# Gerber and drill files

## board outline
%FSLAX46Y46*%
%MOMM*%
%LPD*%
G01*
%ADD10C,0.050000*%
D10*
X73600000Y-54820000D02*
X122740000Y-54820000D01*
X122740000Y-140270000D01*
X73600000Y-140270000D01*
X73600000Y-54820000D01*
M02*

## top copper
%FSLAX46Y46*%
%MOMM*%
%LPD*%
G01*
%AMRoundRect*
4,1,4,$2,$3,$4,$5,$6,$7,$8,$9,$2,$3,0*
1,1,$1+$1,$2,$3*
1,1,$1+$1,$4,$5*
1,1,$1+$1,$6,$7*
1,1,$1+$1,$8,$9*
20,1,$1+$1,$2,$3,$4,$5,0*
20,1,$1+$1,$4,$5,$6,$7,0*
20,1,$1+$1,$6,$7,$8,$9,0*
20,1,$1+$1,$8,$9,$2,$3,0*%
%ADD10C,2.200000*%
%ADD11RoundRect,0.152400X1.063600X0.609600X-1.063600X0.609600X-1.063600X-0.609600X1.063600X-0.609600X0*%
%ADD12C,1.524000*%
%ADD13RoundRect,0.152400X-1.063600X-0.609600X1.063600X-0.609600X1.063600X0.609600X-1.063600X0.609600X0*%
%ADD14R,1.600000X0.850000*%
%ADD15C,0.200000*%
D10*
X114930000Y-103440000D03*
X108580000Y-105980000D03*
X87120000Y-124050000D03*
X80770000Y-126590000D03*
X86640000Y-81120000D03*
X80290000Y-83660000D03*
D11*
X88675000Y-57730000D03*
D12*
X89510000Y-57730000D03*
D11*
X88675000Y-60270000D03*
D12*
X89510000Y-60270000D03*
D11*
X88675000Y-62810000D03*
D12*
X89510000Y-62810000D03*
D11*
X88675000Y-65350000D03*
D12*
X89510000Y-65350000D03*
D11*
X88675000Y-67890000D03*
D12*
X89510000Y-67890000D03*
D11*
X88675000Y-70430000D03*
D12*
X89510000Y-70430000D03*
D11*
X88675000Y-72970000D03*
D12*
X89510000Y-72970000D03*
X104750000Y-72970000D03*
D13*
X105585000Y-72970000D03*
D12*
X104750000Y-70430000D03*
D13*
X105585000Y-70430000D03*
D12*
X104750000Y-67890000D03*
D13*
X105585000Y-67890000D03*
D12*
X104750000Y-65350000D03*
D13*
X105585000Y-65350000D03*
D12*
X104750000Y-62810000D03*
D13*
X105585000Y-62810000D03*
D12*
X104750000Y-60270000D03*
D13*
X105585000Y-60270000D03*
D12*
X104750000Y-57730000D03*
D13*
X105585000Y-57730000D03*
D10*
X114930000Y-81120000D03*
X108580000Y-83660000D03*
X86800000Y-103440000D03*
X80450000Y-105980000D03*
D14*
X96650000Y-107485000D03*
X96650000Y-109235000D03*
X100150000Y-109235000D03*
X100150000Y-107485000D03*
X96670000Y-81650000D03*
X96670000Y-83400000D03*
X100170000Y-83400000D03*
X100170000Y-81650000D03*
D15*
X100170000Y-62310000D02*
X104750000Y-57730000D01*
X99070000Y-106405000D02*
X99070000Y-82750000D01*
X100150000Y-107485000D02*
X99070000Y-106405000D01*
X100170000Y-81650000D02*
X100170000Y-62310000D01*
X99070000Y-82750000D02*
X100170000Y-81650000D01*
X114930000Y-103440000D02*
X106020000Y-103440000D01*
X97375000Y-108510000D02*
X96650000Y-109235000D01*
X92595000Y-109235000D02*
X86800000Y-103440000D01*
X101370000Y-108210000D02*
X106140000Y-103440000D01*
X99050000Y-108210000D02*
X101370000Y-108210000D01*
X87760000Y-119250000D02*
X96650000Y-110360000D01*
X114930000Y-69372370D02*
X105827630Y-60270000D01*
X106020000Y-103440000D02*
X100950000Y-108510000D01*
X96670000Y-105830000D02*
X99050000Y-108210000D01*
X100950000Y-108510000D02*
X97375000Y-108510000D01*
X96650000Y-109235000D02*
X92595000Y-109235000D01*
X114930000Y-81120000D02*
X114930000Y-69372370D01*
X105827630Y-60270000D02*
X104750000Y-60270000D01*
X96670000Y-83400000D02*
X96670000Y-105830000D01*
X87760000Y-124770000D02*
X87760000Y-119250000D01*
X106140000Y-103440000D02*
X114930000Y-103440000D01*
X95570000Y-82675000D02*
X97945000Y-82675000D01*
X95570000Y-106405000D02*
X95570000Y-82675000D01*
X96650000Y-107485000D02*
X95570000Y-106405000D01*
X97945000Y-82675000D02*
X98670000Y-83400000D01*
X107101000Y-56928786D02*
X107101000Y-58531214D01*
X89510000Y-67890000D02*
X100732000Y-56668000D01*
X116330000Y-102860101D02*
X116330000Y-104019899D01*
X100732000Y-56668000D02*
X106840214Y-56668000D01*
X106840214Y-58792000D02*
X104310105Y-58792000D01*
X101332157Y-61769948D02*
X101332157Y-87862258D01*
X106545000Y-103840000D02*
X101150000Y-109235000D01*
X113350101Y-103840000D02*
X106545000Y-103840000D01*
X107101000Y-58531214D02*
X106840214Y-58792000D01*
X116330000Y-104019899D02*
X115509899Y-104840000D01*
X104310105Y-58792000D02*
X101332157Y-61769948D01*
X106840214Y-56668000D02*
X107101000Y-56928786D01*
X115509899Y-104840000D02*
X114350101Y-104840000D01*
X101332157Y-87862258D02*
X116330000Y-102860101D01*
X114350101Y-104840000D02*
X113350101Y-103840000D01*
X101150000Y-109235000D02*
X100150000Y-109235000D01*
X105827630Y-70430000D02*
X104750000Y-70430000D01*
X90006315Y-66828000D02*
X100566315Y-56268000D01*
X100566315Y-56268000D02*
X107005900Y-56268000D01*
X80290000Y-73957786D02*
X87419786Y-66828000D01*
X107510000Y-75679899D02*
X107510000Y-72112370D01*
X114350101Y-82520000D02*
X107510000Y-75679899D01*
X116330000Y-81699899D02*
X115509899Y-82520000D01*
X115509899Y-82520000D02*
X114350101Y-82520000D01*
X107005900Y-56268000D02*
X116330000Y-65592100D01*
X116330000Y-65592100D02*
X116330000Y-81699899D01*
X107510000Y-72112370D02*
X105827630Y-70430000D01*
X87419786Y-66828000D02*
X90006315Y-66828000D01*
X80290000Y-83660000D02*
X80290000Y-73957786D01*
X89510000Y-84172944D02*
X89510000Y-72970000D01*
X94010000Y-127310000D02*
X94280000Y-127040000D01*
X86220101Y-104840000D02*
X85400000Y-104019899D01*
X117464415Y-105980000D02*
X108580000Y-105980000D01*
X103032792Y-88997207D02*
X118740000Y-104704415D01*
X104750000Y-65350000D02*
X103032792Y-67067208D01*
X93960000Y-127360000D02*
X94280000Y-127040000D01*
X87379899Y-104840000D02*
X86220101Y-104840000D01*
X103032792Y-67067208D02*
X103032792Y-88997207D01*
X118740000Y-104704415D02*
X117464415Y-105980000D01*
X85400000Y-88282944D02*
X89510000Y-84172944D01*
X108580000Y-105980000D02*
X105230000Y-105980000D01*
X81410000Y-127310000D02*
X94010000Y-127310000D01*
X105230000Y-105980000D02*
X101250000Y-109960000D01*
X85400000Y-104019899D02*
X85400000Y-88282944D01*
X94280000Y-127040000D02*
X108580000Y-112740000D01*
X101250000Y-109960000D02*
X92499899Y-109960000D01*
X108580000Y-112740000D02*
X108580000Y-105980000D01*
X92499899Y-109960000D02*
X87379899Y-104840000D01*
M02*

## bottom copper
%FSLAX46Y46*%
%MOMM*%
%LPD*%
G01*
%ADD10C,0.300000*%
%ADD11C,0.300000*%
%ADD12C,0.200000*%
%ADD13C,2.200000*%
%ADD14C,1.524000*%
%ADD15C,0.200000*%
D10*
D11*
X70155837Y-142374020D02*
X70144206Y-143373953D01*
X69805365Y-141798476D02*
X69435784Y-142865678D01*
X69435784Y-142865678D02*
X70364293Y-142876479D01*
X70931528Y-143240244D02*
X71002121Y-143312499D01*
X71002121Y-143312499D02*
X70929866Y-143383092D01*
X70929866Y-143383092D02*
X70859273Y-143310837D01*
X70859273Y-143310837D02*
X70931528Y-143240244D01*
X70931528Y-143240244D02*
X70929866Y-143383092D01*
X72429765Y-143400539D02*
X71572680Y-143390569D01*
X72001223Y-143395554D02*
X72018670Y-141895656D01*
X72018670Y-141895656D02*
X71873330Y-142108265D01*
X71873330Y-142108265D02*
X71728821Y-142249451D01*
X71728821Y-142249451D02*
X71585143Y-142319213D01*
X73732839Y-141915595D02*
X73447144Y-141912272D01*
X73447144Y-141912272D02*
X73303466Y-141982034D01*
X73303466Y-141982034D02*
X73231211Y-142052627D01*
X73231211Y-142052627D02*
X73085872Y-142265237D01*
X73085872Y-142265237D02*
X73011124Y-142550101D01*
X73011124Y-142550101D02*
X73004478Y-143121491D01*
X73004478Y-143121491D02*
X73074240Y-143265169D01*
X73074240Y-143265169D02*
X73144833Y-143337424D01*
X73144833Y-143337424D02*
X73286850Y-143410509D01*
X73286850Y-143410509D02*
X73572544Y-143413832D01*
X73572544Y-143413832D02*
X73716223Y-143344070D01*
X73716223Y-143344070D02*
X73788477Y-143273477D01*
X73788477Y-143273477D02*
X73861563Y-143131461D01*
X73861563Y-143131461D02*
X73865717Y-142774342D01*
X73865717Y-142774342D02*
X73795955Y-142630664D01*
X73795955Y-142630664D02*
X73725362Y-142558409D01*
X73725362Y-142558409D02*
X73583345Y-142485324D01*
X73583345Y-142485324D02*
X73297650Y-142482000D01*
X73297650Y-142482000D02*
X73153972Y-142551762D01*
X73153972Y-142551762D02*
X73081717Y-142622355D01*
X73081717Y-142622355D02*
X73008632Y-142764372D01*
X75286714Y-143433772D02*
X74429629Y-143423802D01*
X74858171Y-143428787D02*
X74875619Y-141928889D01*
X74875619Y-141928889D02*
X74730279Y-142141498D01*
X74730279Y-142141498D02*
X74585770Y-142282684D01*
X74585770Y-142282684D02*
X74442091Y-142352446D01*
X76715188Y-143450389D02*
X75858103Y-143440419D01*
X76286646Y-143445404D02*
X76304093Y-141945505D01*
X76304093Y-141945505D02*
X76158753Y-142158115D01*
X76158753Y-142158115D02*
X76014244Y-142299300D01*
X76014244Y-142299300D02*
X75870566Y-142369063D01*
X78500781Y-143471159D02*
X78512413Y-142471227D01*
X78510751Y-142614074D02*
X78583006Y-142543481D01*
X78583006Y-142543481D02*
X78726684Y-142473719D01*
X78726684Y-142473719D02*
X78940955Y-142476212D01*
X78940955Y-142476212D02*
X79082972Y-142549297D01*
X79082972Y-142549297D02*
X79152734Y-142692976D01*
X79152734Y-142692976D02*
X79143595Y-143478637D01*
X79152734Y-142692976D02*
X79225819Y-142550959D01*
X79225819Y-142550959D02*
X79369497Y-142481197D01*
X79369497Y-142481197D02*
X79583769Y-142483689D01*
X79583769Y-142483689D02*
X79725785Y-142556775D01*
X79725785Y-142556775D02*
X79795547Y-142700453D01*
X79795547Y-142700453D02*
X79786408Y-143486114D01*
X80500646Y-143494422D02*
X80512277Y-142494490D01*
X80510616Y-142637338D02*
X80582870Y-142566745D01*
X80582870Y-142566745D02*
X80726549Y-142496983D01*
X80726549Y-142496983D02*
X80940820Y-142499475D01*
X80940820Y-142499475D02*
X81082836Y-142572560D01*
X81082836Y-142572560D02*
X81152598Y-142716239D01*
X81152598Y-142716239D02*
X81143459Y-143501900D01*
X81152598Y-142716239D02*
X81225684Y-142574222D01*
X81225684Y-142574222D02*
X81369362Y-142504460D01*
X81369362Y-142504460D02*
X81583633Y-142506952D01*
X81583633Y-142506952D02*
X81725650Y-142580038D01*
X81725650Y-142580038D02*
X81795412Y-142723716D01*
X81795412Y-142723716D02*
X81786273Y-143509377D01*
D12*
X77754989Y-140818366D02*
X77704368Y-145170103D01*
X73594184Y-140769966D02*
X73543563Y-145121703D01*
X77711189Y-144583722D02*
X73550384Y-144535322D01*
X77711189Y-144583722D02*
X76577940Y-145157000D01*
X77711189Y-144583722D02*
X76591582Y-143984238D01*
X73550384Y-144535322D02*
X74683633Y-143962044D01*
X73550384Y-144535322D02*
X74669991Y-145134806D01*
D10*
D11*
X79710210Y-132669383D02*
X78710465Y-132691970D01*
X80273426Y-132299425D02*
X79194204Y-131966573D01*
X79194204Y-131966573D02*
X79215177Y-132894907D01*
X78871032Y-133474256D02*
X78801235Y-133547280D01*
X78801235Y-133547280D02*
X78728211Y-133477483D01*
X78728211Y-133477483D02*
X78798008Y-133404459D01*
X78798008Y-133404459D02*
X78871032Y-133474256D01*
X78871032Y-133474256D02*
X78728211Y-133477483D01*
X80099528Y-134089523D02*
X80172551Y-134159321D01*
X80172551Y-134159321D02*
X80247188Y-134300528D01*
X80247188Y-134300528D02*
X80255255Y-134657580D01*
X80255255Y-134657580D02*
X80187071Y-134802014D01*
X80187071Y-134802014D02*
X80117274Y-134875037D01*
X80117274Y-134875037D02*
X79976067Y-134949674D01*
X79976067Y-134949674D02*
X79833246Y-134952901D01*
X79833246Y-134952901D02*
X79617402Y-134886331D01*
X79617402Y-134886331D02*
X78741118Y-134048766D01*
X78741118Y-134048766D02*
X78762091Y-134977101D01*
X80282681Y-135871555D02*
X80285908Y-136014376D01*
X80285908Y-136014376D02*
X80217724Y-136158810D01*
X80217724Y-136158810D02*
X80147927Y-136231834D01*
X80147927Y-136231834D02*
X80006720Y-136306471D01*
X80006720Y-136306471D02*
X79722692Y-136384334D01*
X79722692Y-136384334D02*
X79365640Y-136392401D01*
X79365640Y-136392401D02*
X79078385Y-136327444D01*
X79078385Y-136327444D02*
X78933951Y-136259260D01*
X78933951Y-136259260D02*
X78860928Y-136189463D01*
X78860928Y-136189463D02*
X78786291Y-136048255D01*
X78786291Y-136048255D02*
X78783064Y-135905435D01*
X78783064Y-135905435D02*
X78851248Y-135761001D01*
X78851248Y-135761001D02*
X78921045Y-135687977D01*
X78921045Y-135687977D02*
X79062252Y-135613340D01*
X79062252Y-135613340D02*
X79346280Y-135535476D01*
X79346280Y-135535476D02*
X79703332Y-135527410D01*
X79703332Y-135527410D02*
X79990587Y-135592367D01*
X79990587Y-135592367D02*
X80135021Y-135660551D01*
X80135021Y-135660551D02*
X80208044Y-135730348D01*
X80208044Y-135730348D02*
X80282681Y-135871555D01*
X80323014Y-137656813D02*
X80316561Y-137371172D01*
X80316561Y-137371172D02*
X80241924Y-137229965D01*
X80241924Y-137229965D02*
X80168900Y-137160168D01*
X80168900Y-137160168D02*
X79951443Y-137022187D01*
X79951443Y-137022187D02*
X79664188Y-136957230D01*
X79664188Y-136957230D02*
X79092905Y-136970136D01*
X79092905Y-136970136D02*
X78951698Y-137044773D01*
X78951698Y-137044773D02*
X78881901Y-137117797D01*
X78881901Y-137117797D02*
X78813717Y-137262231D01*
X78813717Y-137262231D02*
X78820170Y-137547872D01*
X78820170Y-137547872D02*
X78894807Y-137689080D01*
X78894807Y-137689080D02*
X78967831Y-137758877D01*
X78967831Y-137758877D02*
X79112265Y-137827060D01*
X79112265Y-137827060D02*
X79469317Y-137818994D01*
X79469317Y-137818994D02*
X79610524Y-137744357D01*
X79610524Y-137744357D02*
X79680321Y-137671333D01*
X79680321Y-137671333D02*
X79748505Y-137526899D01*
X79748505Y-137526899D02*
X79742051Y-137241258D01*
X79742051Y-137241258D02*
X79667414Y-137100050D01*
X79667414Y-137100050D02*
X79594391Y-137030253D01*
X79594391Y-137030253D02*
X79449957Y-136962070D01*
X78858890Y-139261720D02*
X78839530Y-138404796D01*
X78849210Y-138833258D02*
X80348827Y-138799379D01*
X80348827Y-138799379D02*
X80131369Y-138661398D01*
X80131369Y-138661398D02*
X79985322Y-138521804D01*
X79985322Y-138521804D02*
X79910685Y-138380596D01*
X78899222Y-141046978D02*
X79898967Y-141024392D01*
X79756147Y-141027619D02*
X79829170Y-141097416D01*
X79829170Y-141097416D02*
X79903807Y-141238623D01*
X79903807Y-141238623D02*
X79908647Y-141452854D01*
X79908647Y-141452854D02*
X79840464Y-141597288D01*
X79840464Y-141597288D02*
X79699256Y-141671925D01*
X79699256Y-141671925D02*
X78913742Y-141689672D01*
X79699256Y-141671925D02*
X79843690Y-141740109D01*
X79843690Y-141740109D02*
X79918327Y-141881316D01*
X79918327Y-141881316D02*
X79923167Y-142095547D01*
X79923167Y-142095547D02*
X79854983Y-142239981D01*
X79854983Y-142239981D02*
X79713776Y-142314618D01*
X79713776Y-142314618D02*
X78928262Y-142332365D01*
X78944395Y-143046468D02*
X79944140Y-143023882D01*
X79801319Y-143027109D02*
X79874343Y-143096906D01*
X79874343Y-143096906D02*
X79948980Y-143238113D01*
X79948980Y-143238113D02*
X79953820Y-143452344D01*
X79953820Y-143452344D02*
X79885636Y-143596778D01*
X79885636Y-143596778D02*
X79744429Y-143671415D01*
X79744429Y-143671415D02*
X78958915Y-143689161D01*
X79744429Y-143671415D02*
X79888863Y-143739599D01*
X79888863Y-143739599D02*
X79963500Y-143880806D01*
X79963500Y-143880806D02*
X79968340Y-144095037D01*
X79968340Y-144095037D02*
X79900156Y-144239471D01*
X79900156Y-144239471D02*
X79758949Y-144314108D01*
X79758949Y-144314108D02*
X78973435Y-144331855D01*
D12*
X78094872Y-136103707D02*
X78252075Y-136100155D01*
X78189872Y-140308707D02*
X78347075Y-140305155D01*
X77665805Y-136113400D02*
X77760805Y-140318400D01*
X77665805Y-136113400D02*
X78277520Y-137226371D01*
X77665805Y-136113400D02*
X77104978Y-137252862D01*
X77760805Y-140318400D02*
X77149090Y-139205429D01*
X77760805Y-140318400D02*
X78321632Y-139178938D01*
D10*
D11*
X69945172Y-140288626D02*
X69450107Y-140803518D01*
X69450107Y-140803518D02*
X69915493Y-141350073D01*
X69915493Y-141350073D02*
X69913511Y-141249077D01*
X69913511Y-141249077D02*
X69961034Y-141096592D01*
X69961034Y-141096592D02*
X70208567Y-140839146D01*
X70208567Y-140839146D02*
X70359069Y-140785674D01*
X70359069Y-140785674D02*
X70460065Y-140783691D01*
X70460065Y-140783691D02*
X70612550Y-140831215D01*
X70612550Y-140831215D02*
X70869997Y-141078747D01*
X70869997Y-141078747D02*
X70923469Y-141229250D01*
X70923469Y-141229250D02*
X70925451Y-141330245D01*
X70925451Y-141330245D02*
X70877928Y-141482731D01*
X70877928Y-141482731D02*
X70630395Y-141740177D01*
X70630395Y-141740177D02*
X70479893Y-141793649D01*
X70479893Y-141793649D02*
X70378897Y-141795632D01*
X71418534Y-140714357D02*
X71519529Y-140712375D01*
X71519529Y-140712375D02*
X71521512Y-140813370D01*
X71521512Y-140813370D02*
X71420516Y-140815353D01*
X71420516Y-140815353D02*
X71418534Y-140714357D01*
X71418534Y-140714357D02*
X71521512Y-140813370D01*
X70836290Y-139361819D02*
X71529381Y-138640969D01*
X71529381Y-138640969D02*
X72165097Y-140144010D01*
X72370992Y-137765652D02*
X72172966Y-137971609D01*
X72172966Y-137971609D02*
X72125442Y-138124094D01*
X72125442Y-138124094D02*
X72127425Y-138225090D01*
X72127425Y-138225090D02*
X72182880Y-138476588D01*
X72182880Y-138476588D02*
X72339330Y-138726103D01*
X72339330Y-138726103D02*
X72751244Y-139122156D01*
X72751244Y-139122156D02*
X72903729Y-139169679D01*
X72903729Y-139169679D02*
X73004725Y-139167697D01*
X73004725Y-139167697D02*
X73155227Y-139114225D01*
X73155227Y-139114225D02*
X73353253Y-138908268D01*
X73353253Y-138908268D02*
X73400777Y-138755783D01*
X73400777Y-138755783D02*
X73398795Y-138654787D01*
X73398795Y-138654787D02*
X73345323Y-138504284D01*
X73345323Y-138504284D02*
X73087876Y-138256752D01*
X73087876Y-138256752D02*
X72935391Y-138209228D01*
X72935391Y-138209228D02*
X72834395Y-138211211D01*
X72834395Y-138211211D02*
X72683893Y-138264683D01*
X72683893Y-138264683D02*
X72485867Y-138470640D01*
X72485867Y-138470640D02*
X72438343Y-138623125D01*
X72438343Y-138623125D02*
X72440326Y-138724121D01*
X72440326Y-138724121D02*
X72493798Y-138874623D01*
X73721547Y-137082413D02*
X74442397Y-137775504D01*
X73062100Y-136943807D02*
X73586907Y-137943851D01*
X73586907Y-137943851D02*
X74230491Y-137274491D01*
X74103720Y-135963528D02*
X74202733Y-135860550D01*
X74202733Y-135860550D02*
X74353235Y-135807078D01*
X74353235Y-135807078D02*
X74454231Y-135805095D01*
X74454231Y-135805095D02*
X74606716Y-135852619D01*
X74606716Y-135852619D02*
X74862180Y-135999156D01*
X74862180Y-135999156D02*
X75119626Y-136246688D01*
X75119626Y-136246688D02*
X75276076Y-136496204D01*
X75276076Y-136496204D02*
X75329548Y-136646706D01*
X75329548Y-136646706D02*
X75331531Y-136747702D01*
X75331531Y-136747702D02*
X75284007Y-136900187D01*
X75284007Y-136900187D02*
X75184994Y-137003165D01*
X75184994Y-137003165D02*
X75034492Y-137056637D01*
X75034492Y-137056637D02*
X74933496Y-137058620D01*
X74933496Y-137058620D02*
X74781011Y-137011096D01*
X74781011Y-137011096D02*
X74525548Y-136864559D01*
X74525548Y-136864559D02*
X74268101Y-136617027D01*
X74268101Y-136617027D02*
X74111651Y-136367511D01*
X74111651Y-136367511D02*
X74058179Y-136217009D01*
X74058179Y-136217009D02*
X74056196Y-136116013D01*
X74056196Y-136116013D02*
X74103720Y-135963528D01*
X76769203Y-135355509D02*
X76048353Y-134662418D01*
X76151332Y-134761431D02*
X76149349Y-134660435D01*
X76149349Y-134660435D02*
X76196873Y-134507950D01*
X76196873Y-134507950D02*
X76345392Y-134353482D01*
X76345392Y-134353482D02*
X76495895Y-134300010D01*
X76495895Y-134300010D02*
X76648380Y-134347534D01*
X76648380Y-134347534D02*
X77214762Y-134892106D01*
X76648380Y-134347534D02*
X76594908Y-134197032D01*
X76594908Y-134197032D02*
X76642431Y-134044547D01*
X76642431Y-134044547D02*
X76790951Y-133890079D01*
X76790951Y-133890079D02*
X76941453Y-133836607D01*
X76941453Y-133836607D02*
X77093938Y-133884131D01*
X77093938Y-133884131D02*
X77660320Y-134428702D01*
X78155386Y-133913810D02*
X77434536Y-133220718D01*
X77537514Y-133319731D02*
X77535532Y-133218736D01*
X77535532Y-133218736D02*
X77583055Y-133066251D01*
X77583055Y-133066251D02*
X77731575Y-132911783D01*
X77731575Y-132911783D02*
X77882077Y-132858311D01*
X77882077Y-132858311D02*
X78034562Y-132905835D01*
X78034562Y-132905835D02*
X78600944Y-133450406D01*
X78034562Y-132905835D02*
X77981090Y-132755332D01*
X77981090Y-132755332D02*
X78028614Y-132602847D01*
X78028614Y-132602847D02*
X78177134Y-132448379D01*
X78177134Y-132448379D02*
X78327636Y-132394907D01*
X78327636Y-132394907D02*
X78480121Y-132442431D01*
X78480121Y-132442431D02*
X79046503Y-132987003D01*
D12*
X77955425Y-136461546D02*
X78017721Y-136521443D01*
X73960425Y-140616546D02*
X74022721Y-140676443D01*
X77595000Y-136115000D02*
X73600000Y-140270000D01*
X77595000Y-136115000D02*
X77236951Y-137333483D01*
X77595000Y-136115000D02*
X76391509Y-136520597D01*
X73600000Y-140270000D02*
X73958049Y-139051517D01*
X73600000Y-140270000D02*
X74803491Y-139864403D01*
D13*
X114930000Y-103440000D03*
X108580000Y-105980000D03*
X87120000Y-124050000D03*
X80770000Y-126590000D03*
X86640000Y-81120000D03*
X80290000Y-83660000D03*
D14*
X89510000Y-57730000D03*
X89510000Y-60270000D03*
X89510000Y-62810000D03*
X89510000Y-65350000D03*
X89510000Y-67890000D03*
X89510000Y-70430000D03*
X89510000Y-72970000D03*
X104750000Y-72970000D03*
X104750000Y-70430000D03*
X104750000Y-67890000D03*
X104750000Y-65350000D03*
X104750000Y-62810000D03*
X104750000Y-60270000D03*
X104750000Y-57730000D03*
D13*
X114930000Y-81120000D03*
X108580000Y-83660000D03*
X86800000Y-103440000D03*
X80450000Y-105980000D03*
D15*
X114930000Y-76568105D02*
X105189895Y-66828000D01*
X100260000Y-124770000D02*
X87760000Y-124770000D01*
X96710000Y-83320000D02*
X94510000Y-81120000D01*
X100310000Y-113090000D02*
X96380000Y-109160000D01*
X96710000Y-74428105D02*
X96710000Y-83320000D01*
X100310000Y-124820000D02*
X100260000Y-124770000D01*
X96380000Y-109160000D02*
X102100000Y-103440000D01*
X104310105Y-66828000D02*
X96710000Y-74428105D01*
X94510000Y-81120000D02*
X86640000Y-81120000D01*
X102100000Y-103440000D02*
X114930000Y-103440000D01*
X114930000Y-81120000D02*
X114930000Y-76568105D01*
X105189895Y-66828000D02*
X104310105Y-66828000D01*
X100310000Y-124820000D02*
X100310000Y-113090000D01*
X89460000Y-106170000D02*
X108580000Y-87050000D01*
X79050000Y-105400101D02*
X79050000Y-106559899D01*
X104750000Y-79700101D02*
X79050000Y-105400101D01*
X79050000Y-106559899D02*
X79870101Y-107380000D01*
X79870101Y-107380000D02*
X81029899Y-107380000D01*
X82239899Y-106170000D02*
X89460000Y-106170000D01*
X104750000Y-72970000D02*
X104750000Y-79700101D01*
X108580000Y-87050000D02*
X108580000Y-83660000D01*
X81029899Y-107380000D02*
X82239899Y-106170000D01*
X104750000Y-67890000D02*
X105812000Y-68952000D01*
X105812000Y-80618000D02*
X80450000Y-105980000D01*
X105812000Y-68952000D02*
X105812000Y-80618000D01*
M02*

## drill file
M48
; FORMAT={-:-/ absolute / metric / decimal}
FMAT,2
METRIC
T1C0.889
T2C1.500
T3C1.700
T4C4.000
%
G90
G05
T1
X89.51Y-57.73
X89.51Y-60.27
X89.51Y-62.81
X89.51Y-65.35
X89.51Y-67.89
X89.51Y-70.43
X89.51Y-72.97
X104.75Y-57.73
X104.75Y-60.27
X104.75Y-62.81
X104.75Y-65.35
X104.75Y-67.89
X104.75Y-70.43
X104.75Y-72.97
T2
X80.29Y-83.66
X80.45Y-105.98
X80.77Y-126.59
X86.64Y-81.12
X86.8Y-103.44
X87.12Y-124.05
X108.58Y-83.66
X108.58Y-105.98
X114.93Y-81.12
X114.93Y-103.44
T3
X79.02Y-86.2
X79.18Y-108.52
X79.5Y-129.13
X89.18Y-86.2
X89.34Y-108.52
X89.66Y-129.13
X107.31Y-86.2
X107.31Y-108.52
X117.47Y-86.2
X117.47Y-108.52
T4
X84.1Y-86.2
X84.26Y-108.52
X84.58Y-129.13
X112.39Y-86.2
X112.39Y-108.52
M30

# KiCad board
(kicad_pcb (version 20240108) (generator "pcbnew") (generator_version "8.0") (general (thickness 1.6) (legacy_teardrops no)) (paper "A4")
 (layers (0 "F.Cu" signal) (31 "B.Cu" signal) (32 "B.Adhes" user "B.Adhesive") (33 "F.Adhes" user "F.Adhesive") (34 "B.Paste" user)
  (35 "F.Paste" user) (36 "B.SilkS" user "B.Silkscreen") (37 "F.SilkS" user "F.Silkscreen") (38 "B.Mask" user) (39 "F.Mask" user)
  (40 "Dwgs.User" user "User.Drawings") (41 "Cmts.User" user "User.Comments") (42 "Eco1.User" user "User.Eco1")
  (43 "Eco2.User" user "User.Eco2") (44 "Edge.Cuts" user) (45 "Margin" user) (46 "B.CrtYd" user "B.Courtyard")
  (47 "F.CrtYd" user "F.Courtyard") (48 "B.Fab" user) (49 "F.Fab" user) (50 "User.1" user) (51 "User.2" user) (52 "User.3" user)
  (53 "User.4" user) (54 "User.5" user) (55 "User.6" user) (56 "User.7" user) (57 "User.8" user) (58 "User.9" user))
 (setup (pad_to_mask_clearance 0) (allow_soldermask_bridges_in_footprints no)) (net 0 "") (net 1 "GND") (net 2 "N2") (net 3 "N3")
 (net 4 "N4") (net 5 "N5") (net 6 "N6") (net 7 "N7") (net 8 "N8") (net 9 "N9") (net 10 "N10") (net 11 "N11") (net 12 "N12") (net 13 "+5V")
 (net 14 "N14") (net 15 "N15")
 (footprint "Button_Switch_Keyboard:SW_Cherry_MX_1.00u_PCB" (layer "F.Cu") (at 114.93 103.44)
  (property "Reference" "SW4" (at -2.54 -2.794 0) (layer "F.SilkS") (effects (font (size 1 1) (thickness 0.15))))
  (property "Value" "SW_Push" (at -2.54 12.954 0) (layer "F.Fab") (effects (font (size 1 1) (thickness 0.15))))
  (pad "" np_thru_hole circle (at -7.62 5.08) (size 1.7 1.7) (drill 1.7) (layers "*.Cu" "*.Mask"))
  (pad "" np_thru_hole circle (at -2.54 5.08) (size 4 4) (drill 4) (layers "*.Cu" "*.Mask"))
  (pad "" np_thru_hole circle (at 2.54 5.08) (size 1.7 1.7) (drill 1.7) (layers "*.Cu" "*.Mask"))
  (pad "1" thru_hole circle (at 0 0) (size 2.2 2.2) (drill 1.5) (layers "*.Cu" "*.Mask") (remove_unused_layers no) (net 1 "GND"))
  (pad "2" thru_hole circle (at -6.35 2.54) (size 2.2 2.2) (drill 1.5) (layers "*.Cu" "*.Mask") (remove_unused_layers no) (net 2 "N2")))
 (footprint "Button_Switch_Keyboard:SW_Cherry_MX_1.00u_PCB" (layer "F.Cu") (at 87.12 124.05)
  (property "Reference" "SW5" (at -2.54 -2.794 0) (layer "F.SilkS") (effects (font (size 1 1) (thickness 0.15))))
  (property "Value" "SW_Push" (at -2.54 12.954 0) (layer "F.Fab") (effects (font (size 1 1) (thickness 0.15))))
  (pad "" np_thru_hole circle (at -7.62 5.08) (size 1.7 1.7) (drill 1.7) (layers "*.Cu" "*.Mask"))
  (pad "" np_thru_hole circle (at -2.54 5.08) (size 4 4) (drill 4) (layers "*.Cu" "*.Mask"))
  (pad "" np_thru_hole circle (at 2.54 5.08) (size 1.7 1.7) (drill 1.7) (layers "*.Cu" "*.Mask"))
  (pad "1" thru_hole circle (at 0 0) (size 2.2 2.2) (drill 1.5) (layers "*.Cu" "*.Mask") (remove_unused_layers no) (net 1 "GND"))
  (pad "2" thru_hole circle (at -6.35 2.54) (size 2.2 2.2) (drill 1.5) (layers "*.Cu" "*.Mask") (remove_unused_layers no) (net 2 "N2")))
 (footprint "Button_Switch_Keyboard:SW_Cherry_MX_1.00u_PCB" (layer "F.Cu") (at 86.64 81.12)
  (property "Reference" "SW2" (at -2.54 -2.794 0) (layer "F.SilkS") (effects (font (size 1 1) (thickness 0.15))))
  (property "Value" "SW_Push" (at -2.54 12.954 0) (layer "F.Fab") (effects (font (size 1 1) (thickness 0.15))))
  (pad "" np_thru_hole circle (at -7.62 5.08) (size 1.7 1.7) (drill 1.7) (layers "*.Cu" "*.Mask"))
  (pad "" np_thru_hole circle (at -2.54 5.08) (size 4 4) (drill 4) (layers "*.Cu" "*.Mask"))
  (pad "" np_thru_hole circle (at 2.54 5.08) (size 1.7 1.7) (drill 1.7) (layers "*.Cu" "*.Mask"))
  (pad "1" thru_hole circle (at 0 0) (size 2.2 2.2) (drill 1.5) (layers "*.Cu" "*.Mask") (remove_unused_layers no) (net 1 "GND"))
  (pad "2" thru_hole circle (at -6.35 2.54) (size 2.2 2.2) (drill 1.5) (layers "*.Cu" "*.Mask") (remove_unused_layers no) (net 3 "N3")))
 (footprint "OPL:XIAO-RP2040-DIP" (layer "F.Cu") (at 97.13 65.35)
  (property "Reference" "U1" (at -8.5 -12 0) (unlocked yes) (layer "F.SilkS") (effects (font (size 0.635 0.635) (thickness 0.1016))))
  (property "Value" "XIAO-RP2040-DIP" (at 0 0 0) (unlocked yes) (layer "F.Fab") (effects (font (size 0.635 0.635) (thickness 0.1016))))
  (pad "1" smd roundrect (at -8.455 -7.62 180) (size 2.432 1.524) (layers "F.Cu" "F.Mask") (roundrect_rratio 0.1) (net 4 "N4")
   (thermal_bridge_angle 45))
  (pad "1" thru_hole circle (at -7.62 -7.62 180) (size 1.524 1.524) (drill 0.889) (layers "*.Cu" "*.Mask") (remove_unused_layers no)
   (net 4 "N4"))
  (pad "2" smd roundrect (at -8.455 -5.08 180) (size 2.432 1.524) (layers "F.Cu" "F.Mask") (roundrect_rratio 0.1) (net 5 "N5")
   (thermal_bridge_angle 45))
  (pad "2" thru_hole circle (at -7.62 -5.08 180) (size 1.524 1.524) (drill 0.889) (layers "*.Cu" "*.Mask") (remove_unused_layers no)
   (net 5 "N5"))
  (pad "3" smd roundrect (at -8.455 -2.54 180) (size 2.432 1.524) (layers "F.Cu" "F.Mask") (roundrect_rratio 0.1) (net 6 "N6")
   (thermal_bridge_angle 45))
  (pad "3" thru_hole circle (at -7.62 -2.54 180) (size 1.524 1.524) (drill 0.889) (layers "*.Cu" "*.Mask") (remove_unused_layers no)
   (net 6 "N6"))
  (pad "4" smd roundrect (at -8.455 0 180) (size 2.432 1.524) (layers "F.Cu" "F.Mask") (roundrect_rratio 0.1) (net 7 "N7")
   (thermal_bridge_angle 45))
  (pad "4" thru_hole circle (at -7.62 0 180) (size 1.524 1.524) (drill 0.889) (layers "*.Cu" "*.Mask") (remove_unused_layers no)
   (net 7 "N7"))
  (pad "5" smd roundrect (at -8.455 2.54 180) (size 2.432 1.524) (layers "F.Cu" "F.Mask") (roundrect_rratio 0.1) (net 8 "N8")
   (thermal_bridge_angle 45))
  (pad "5" thru_hole circle (at -7.62 2.54 180) (size 1.524 1.524) (drill 0.889) (layers "*.Cu" "*.Mask") (remove_unused_layers no)
   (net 8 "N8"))
  (pad "6" smd roundrect (at -8.455 5.08 180) (size 2.432 1.524) (layers "F.Cu" "F.Mask") (roundrect_rratio 0.1) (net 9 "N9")
   (thermal_bridge_angle 45))
  (pad "6" thru_hole circle (at -7.62 5.08 180) (size 1.524 1.524) (drill 0.889) (layers "*.Cu" "*.Mask") (remove_unused_layers no)
   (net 9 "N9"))
  (pad "7" smd roundrect (at -8.455 7.62 180) (size 2.432 1.524) (layers "F.Cu" "F.Mask") (roundrect_rratio 0.1) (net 2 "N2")
   (thermal_bridge_angle 45))
  (pad "7" thru_hole circle (at -7.62 7.62 180) (size 1.524 1.524) (drill 0.889) (layers "*.Cu" "*.Mask") (remove_unused_layers no)
   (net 2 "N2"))
  (pad "8" thru_hole circle (at 7.62 7.62) (size 1.524 1.524) (drill 0.889) (layers "*.Cu" "*.Mask") (remove_unused_layers no)
   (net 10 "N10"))
  (pad "8" smd roundrect (at 8.455 7.62) (size 2.432 1.524) (layers "F.Cu" "F.Mask") (roundrect_rratio 0.1) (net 10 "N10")
   (thermal_bridge_angle 45))
  (pad "9" thru_hole circle (at 7.62 5.08) (size 1.524 1.524) (drill 0.889) (layers "*.Cu" "*.Mask") (remove_unused_layers no) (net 3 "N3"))
  (pad "9" smd roundrect (at 8.455 5.08) (size 2.432 1.524) (layers "F.Cu" "F.Mask") (roundrect_rratio 0.1) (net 3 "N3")
   (thermal_bridge_angle 45))
  (pad "10" thru_hole circle (at 7.62 2.54) (size 1.524 1.524) (drill 0.889) (layers "*.Cu" "*.Mask") (remove_unused_layers no)
   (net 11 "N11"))
  (pad "10" smd roundrect (at 8.455 2.54) (size 2.432 1.524) (layers "F.Cu" "F.Mask") (roundrect_rratio 0.1) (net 11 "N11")
   (thermal_bridge_angle 45))
  (pad "11" thru_hole circle (at 7.62 0) (size 1.524 1.524) (drill 0.889) (layers "*.Cu" "*.Mask") (remove_unused_layers no) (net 2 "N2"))
  (pad "11" smd roundrect (at 8.455 0) (size 2.432 1.524) (layers "F.Cu" "F.Mask") (roundrect_rratio 0.1) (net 2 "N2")
   (thermal_bridge_angle 45))
  (pad "12" thru_hole circle (at 7.62 -2.54) (size 1.524 1.524) (drill 0.889) (layers "*.Cu" "*.Mask") (remove_unused_layers no)
   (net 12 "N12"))
  (pad "12" smd roundrect (at 8.455 -2.54) (size 2.432 1.524) (layers "F.Cu" "F.Mask") (roundrect_rratio 0.1) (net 12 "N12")
   (thermal_bridge_angle 45))
  (pad "13" thru_hole circle (at 7.62 -5.08) (size 1.524 1.524) (drill 0.889) (layers "*.Cu" "*.Mask") (remove_unused_layers no)
   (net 1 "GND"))
  (pad "13" smd roundrect (at 8.455 -5.08) (size 2.432 1.524) (layers "F.Cu" "F.Mask") (roundrect_rratio 0.1) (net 1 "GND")
   (thermal_bridge_angle 45))
  (pad "14" thru_hole circle (at 7.62 -7.62) (size 1.524 1.524) (drill 0.889) (layers "*.Cu" "*.Mask") (remove_unused_layers no)
   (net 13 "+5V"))
  (pad "14" smd roundrect (at 8.455 -7.62) (size 2.432 1.524) (layers "F.Cu" "F.Mask") (roundrect_rratio 0.1) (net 13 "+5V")
   (thermal_bridge_angle 45)))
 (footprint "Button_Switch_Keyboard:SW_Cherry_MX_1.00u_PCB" (layer "F.Cu") (at 114.93 81.12)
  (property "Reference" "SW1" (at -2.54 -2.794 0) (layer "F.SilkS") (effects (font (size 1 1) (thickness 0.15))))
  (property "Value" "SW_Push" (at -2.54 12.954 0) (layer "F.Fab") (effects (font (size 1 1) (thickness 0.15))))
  (pad "" np_thru_hole circle (at -7.62 5.08) (size 1.7 1.7) (drill 1.7) (layers "*.Cu" "*.Mask"))
  (pad "" np_thru_hole circle (at -2.54 5.08) (size 4 4) (drill 4) (layers "*.Cu" "*.Mask"))
  (pad "" np_thru_hole circle (at 2.54 5.08) (size 1.7 1.7) (drill 1.7) (layers "*.Cu" "*.Mask"))
  (pad "1" thru_hole circle (at 0 0) (size 2.2 2.2) (drill 1.5) (layers "*.Cu" "*.Mask") (remove_unused_layers no) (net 1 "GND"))
  (pad "2" thru_hole circle (at -6.35 2.54) (size 2.2 2.2) (drill 1.5) (layers "*.Cu" "*.Mask") (remove_unused_layers no) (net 10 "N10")))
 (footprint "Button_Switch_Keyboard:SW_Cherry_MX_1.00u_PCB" (layer "F.Cu") (at 86.8 103.44)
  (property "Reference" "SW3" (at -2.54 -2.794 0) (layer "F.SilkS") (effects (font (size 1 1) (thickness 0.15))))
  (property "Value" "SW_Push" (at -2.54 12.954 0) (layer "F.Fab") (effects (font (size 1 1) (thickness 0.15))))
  (pad "" np_thru_hole circle (at -7.62 5.08) (size 1.7 1.7) (drill 1.7) (layers "*.Cu" "*.Mask"))
  (pad "" np_thru_hole circle (at -2.54 5.08) (size 4 4) (drill 4) (layers "*.Cu" "*.Mask"))
  (pad "" np_thru_hole circle (at 2.54 5.08) (size 1.7 1.7) (drill 1.7) (layers "*.Cu" "*.Mask"))
  (pad "1" thru_hole circle (at 0 0) (size 2.2 2.2) (drill 1.5) (layers "*.Cu" "*.Mask") (remove_unused_layers no) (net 1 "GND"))
  (pad "2" thru_hole circle (at -6.35 2.54) (size 2.2 2.2) (drill 1.5) (layers "*.Cu" "*.Mask") (remove_unused_layers no) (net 11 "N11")))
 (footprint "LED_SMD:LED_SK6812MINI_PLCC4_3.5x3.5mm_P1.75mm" (layer "F.Cu") (at 98.4 108.36)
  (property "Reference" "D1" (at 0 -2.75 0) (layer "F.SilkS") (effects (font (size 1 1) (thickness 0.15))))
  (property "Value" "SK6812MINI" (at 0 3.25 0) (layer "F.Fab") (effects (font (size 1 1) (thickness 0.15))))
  (pad "1" smd rect (at -1.75 -0.875) (size 1.6 0.85) (layers "F.Cu" "F.Paste" "F.Mask") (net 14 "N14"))
  (pad "2" smd rect (at -1.75 0.875) (size 1.6 0.85) (layers "F.Cu" "F.Paste" "F.Mask") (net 1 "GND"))
  (pad "3" smd rect (at 1.75 0.875) (size 1.6 0.85) (layers "F.Cu" "F.Paste" "F.Mask") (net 8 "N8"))
  (pad "4" smd rect (at 1.75 -0.875) (size 1.6 0.85) (layers "F.Cu" "F.Paste" "F.Mask") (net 13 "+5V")))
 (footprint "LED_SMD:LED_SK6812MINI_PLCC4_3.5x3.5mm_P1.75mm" (layer "F.Cu") (at 98.42 82.525)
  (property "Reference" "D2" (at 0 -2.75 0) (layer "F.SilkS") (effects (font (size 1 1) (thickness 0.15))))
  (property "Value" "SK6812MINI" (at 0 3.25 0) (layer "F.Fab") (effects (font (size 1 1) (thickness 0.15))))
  (pad "1" smd rect (at -1.75 -0.875) (size 1.6 0.85) (layers "F.Cu" "F.Paste" "F.Mask") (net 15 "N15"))
  (pad "2" smd rect (at -1.75 0.875) (size 1.6 0.85) (layers "F.Cu" "F.Paste" "F.Mask") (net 1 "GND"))
  (pad "3" smd rect (at 1.75 0.875) (size 1.6 0.85) (layers "F.Cu" "F.Paste" "F.Mask") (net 14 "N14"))
  (pad "4" smd rect (at 1.75 -0.875) (size 1.6 0.85) (layers "F.Cu" "F.Paste" "F.Mask") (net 13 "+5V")))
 (gr_rect (start 73.6 54.82) (end 122.74 140.27) (stroke (width 0.05) (type default)) (fill none) (layer "Edge.Cuts"))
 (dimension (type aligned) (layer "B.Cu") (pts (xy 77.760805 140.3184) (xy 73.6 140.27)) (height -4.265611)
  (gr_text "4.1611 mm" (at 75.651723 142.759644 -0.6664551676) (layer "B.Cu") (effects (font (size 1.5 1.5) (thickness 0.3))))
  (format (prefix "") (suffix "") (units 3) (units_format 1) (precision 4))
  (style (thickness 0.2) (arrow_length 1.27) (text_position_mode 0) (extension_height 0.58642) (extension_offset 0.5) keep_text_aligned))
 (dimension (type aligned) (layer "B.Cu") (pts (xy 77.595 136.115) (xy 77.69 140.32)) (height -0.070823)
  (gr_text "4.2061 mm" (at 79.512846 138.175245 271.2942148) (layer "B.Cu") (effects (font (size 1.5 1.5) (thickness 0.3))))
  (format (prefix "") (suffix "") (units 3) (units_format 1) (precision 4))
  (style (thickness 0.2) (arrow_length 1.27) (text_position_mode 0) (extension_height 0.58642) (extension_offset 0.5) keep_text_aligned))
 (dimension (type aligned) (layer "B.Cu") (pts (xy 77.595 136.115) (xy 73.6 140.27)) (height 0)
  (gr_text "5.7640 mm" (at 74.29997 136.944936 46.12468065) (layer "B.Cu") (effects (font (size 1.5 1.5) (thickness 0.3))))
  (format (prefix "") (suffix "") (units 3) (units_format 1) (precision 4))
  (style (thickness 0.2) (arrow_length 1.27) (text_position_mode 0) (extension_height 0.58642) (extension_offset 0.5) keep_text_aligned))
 (segment (start 100.17 62.31) (end 104.75 57.73) (width 0.2) (layer "F.Cu") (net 13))
 (segment (start 99.07 106.405) (end 99.07 82.75) (width 0.2) (layer "F.Cu") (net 13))
 (segment (start 100.15 107.485) (end 99.07 106.405) (width 0.2) (layer "F.Cu") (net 13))
 (segment (start 100.17 81.65) (end 100.17 62.31) (width 0.2) (layer "F.Cu") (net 13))
 (segment (start 99.07 82.75) (end 100.17 81.65) (width 0.2) (layer "F.Cu") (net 13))
 (segment (start 114.93 103.44) (end 106.02 103.44) (width 0.2) (layer "F.Cu") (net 1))
 (segment (start 97.375 108.51) (end 96.65 109.235) (width 0.2) (layer "F.Cu") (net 1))
 (segment (start 92.595 109.235) (end 86.8 103.44) (width 0.2) (layer "F.Cu") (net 1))
 (segment (start 101.37 108.21) (end 106.14 103.44) (width 0.2) (layer "F.Cu") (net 1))
 (segment (start 99.05 108.21) (end 101.37 108.21) (width 0.2) (layer "F.Cu") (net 1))
 (segment (start 87.76 119.25) (end 96.65 110.36) (width 0.2) (layer "F.Cu") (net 1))
 (segment (start 114.93 69.37237) (end 105.82763 60.27) (width 0.2) (layer "F.Cu") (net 1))
 (segment (start 106.02 103.44) (end 100.95 108.51) (width 0.2) (layer "F.Cu") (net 1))
 (segment (start 96.67 105.83) (end 99.05 108.21) (width 0.2) (layer "F.Cu") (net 1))
 (segment (start 100.95 108.51) (end 97.375 108.51) (width 0.2) (layer "F.Cu") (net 1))
 (segment (start 96.65 109.235) (end 92.595 109.235) (width 0.2) (layer "F.Cu") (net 1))
 (segment (start 114.93 81.12) (end 114.93 69.37237) (width 0.2) (layer "F.Cu") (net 1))
 (segment (start 105.82763 60.27) (end 104.75 60.27) (width 0.2) (layer "F.Cu") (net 1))
 (segment (start 96.67 83.4) (end 96.67 105.83) (width 0.2) (layer "F.Cu") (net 1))
 (segment (start 87.76 124.77) (end 87.76 119.25) (width 0.2) (layer "F.Cu") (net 1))
 (segment (start 106.14 103.44) (end 114.93 103.44) (width 0.2) (layer "F.Cu") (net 1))
 (segment (start 114.93 76.568105) (end 105.189895 66.828) (width 0.2) (layer "B.Cu") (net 1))
 (segment (start 100.26 124.77) (end 87.76 124.77) (width 0.2) (layer "B.Cu") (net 1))
 (segment (start 96.71 83.32) (end 94.51 81.12) (width 0.2) (layer "B.Cu") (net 1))
 (segment (start 100.31 113.09) (end 96.38 109.16) (width 0.2) (layer "B.Cu") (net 1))
 (segment (start 96.71 74.428105) (end 96.71 83.32) (width 0.2) (layer "B.Cu") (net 1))
 (segment (start 100.31 124.82) (end 100.26 124.77) (width 0.2) (layer "B.Cu") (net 1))
 (segment (start 96.38 109.16) (end 102.1 103.44) (width 0.2) (layer "B.Cu") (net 1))
 (segment (start 104.310105 66.828) (end 96.71 74.428105) (width 0.2) (layer "B.Cu") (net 1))
 (segment (start 94.51 81.12) (end 86.64 81.12) (width 0.2) (layer "B.Cu") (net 1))
 (segment (start 102.1 103.44) (end 114.93 103.44) (width 0.2) (layer "B.Cu") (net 1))
 (segment (start 114.93 81.12) (end 114.93 76.568105) (width 0.2) (layer "B.Cu") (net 1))
 (segment (start 105.189895 66.828) (end 104.310105 66.828) (width 0.2) (layer "B.Cu") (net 1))
 (segment (start 100.31 124.82) (end 100.31 113.09) (width 0.2) (layer "B.Cu") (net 1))
 (segment (start 95.57 82.675) (end 97.945 82.675) (width 0.2) (layer "F.Cu") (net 14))
 (segment (start 95.57 106.405) (end 95.57 82.675) (width 0.2) (layer "F.Cu") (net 14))
 (segment (start 96.65 107.485) (end 95.57 106.405) (width 0.2) (layer "F.Cu") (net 14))
 (segment (start 97.945 82.675) (end 98.67 83.4) (width 0.2) (layer "F.Cu") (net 14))
 (segment (start 107.101 56.928786) (end 107.101 58.531214) (width 0.2) (layer "F.Cu") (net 8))
 (segment (start 89.51 67.89) (end 100.732 56.668) (width 0.2) (layer "F.Cu") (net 8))
 (segment (start 116.33 102.860101) (end 116.33 104.019899) (width 0.2) (layer "F.Cu") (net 8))
 (segment (start 100.732 56.668) (end 106.840214 56.668) (width 0.2) (layer "F.Cu") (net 8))
 (segment (start 106.840214 58.792) (end 104.310105 58.792) (width 0.2) (layer "F.Cu") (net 8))
 (segment (start 101.332157 61.769948) (end 101.332157 87.862258) (width 0.2) (layer "F.Cu") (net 8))
 (segment (start 106.545 103.84) (end 101.15 109.235) (width 0.2) (layer "F.Cu") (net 8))
 (segment (start 113.350101 103.84) (end 106.545 103.84) (width 0.2) (layer "F.Cu") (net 8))
 (segment (start 107.101 58.531214) (end 106.840214 58.792) (width 0.2) (layer "F.Cu") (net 8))
 (segment (start 116.33 104.019899) (end 115.509899 104.84) (width 0.2) (layer "F.Cu") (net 8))
 (segment (start 104.310105 58.792) (end 101.332157 61.769948) (width 0.2) (layer "F.Cu") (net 8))
 (segment (start 106.840214 56.668) (end 107.101 56.928786) (width 0.2) (layer "F.Cu") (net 8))
 (segment (start 115.509899 104.84) (end 114.350101 104.84) (width 0.2) (layer "F.Cu") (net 8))
 (segment (start 101.332157 87.862258) (end 116.33 102.860101) (width 0.2) (layer "F.Cu") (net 8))
 (segment (start 114.350101 104.84) (end 113.350101 103.84) (width 0.2) (layer "F.Cu") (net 8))
 (segment (start 101.15 109.235) (end 100.15 109.235) (width 0.2) (layer "F.Cu") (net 8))
 (segment (start 89.46 106.17) (end 108.58 87.05) (width 0.2) (layer "B.Cu") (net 10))
 (segment (start 79.05 105.400101) (end 79.05 106.559899) (width 0.2) (layer "B.Cu") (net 10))
 (segment (start 104.75 79.700101) (end 79.05 105.400101) (width 0.2) (layer "B.Cu") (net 10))
 (segment (start 79.05 106.559899) (end 79.870101 107.38) (width 0.2) (layer "B.Cu") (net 10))
 (segment (start 79.870101 107.38) (end 81.029899 107.38) (width 0.2) (layer "B.Cu") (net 10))
 (segment (start 82.239899 106.17) (end 89.46 106.17) (width 0.2) (layer "B.Cu") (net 10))
 (segment (start 104.75 72.97) (end 104.75 79.700101) (width 0.2) (layer "B.Cu") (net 10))
 (segment (start 108.58 87.05) (end 108.58 83.66) (width 0.2) (layer "B.Cu") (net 10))
 (segment (start 81.029899 107.38) (end 82.239899 106.17) (width 0.2) (layer "B.Cu") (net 10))
 (segment (start 105.82763 70.43) (end 104.75 70.43) (width 0.2) (layer "F.Cu") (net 3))
 (segment (start 90.006315 66.828) (end 100.566315 56.268) (width 0.2) (layer "F.Cu") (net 3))
 (segment (start 100.566315 56.268) (end 107.0059 56.268) (width 0.2) (layer "F.Cu") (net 3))
 (segment (start 80.29 73.957786) (end 87.419786 66.828) (width 0.2) (layer "F.Cu") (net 3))
 (segment (start 107.51 75.679899) (end 107.51 72.11237) (width 0.2) (layer "F.Cu") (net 3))
 (segment (start 114.350101 82.52) (end 107.51 75.679899) (width 0.2) (layer "F.Cu") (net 3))
 (segment (start 116.33 81.699899) (end 115.509899 82.52) (width 0.2) (layer "F.Cu") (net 3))
 (segment (start 115.509899 82.52) (end 114.350101 82.52) (width 0.2) (layer "F.Cu") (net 3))
 (segment (start 107.0059 56.268) (end 116.33 65.5921) (width 0.2) (layer "F.Cu") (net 3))
 (segment (start 116.33 65.5921) (end 116.33 81.699899) (width 0.2) (layer "F.Cu") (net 3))
 (segment (start 107.51 72.11237) (end 105.82763 70.43) (width 0.2) (layer "F.Cu") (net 3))
 (segment (start 87.419786 66.828) (end 90.006315 66.828) (width 0.2) (layer "F.Cu") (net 3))
 (segment (start 80.29 83.66) (end 80.29 73.957786) (width 0.2) (layer "F.Cu") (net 3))
 (segment (start 104.75 67.89) (end 105.812 68.952) (width 0.2) (layer "B.Cu") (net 11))
 (segment (start 105.812 80.618) (end 80.45 105.98) (width 0.2) (layer "B.Cu") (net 11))
 (segment (start 105.812 68.952) (end 105.812 80.618) (width 0.2) (layer "B.Cu") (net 11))
 (segment (start 89.51 84.172944) (end 89.51 72.97) (width 0.2) (layer "F.Cu") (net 2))
 (segment (start 94.01 127.31) (end 94.28 127.04) (width 0.2) (layer "F.Cu") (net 2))
 (segment (start 86.220101 104.84) (end 85.4 104.019899) (width 0.2) (layer "F.Cu") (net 2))
 (segment (start 117.464415 105.98) (end 108.58 105.98) (width 0.2) (layer "F.Cu") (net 2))
 (segment (start 103.032792 88.997207) (end 118.74 104.704415) (width 0.2) (layer "F.Cu") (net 2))
 (segment (start 104.75 65.35) (end 103.032792 67.067208) (width 0.2) (layer "F.Cu") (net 2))
 (segment (start 93.96 127.36) (end 94.28 127.04) (width 0.2) (layer "F.Cu") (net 2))
 (segment (start 87.379899 104.84) (end 86.220101 104.84) (width 0.2) (layer "F.Cu") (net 2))
 (segment (start 103.032792 67.067208) (end 103.032792 88.997207) (width 0.2) (layer "F.Cu") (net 2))
 (segment (start 118.74 104.704415) (end 117.464415 105.98) (width 0.2) (layer "F.Cu") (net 2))
 (segment (start 85.4 88.282944) (end 89.51 84.172944) (width 0.2) (layer "F.Cu") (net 2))
 (segment (start 108.58 105.98) (end 105.23 105.98) (width 0.2) (layer "F.Cu") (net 2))
 (segment (start 81.41 127.31) (end 94.01 127.31) (width 0.2) (layer "F.Cu") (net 2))
 (segment (start 105.23 105.98) (end 101.25 109.96) (width 0.2) (layer "F.Cu") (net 2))
 (segment (start 85.4 104.019899) (end 85.4 88.282944) (width 0.2) (layer "F.Cu") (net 2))
 (segment (start 94.28 127.04) (end 108.58 112.74) (width 0.2) (layer "F.Cu") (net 2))
 (segment (start 101.25 109.96) (end 92.499899 109.96) (width 0.2) (layer "F.Cu") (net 2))
 (segment (start 108.58 112.74) (end 108.58 105.98) (width 0.2) (layer "F.Cu") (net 2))
 (segment (start 92.499899 109.96) (end 87.379899 104.84) (width 0.2) (layer "F.Cu") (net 2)))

